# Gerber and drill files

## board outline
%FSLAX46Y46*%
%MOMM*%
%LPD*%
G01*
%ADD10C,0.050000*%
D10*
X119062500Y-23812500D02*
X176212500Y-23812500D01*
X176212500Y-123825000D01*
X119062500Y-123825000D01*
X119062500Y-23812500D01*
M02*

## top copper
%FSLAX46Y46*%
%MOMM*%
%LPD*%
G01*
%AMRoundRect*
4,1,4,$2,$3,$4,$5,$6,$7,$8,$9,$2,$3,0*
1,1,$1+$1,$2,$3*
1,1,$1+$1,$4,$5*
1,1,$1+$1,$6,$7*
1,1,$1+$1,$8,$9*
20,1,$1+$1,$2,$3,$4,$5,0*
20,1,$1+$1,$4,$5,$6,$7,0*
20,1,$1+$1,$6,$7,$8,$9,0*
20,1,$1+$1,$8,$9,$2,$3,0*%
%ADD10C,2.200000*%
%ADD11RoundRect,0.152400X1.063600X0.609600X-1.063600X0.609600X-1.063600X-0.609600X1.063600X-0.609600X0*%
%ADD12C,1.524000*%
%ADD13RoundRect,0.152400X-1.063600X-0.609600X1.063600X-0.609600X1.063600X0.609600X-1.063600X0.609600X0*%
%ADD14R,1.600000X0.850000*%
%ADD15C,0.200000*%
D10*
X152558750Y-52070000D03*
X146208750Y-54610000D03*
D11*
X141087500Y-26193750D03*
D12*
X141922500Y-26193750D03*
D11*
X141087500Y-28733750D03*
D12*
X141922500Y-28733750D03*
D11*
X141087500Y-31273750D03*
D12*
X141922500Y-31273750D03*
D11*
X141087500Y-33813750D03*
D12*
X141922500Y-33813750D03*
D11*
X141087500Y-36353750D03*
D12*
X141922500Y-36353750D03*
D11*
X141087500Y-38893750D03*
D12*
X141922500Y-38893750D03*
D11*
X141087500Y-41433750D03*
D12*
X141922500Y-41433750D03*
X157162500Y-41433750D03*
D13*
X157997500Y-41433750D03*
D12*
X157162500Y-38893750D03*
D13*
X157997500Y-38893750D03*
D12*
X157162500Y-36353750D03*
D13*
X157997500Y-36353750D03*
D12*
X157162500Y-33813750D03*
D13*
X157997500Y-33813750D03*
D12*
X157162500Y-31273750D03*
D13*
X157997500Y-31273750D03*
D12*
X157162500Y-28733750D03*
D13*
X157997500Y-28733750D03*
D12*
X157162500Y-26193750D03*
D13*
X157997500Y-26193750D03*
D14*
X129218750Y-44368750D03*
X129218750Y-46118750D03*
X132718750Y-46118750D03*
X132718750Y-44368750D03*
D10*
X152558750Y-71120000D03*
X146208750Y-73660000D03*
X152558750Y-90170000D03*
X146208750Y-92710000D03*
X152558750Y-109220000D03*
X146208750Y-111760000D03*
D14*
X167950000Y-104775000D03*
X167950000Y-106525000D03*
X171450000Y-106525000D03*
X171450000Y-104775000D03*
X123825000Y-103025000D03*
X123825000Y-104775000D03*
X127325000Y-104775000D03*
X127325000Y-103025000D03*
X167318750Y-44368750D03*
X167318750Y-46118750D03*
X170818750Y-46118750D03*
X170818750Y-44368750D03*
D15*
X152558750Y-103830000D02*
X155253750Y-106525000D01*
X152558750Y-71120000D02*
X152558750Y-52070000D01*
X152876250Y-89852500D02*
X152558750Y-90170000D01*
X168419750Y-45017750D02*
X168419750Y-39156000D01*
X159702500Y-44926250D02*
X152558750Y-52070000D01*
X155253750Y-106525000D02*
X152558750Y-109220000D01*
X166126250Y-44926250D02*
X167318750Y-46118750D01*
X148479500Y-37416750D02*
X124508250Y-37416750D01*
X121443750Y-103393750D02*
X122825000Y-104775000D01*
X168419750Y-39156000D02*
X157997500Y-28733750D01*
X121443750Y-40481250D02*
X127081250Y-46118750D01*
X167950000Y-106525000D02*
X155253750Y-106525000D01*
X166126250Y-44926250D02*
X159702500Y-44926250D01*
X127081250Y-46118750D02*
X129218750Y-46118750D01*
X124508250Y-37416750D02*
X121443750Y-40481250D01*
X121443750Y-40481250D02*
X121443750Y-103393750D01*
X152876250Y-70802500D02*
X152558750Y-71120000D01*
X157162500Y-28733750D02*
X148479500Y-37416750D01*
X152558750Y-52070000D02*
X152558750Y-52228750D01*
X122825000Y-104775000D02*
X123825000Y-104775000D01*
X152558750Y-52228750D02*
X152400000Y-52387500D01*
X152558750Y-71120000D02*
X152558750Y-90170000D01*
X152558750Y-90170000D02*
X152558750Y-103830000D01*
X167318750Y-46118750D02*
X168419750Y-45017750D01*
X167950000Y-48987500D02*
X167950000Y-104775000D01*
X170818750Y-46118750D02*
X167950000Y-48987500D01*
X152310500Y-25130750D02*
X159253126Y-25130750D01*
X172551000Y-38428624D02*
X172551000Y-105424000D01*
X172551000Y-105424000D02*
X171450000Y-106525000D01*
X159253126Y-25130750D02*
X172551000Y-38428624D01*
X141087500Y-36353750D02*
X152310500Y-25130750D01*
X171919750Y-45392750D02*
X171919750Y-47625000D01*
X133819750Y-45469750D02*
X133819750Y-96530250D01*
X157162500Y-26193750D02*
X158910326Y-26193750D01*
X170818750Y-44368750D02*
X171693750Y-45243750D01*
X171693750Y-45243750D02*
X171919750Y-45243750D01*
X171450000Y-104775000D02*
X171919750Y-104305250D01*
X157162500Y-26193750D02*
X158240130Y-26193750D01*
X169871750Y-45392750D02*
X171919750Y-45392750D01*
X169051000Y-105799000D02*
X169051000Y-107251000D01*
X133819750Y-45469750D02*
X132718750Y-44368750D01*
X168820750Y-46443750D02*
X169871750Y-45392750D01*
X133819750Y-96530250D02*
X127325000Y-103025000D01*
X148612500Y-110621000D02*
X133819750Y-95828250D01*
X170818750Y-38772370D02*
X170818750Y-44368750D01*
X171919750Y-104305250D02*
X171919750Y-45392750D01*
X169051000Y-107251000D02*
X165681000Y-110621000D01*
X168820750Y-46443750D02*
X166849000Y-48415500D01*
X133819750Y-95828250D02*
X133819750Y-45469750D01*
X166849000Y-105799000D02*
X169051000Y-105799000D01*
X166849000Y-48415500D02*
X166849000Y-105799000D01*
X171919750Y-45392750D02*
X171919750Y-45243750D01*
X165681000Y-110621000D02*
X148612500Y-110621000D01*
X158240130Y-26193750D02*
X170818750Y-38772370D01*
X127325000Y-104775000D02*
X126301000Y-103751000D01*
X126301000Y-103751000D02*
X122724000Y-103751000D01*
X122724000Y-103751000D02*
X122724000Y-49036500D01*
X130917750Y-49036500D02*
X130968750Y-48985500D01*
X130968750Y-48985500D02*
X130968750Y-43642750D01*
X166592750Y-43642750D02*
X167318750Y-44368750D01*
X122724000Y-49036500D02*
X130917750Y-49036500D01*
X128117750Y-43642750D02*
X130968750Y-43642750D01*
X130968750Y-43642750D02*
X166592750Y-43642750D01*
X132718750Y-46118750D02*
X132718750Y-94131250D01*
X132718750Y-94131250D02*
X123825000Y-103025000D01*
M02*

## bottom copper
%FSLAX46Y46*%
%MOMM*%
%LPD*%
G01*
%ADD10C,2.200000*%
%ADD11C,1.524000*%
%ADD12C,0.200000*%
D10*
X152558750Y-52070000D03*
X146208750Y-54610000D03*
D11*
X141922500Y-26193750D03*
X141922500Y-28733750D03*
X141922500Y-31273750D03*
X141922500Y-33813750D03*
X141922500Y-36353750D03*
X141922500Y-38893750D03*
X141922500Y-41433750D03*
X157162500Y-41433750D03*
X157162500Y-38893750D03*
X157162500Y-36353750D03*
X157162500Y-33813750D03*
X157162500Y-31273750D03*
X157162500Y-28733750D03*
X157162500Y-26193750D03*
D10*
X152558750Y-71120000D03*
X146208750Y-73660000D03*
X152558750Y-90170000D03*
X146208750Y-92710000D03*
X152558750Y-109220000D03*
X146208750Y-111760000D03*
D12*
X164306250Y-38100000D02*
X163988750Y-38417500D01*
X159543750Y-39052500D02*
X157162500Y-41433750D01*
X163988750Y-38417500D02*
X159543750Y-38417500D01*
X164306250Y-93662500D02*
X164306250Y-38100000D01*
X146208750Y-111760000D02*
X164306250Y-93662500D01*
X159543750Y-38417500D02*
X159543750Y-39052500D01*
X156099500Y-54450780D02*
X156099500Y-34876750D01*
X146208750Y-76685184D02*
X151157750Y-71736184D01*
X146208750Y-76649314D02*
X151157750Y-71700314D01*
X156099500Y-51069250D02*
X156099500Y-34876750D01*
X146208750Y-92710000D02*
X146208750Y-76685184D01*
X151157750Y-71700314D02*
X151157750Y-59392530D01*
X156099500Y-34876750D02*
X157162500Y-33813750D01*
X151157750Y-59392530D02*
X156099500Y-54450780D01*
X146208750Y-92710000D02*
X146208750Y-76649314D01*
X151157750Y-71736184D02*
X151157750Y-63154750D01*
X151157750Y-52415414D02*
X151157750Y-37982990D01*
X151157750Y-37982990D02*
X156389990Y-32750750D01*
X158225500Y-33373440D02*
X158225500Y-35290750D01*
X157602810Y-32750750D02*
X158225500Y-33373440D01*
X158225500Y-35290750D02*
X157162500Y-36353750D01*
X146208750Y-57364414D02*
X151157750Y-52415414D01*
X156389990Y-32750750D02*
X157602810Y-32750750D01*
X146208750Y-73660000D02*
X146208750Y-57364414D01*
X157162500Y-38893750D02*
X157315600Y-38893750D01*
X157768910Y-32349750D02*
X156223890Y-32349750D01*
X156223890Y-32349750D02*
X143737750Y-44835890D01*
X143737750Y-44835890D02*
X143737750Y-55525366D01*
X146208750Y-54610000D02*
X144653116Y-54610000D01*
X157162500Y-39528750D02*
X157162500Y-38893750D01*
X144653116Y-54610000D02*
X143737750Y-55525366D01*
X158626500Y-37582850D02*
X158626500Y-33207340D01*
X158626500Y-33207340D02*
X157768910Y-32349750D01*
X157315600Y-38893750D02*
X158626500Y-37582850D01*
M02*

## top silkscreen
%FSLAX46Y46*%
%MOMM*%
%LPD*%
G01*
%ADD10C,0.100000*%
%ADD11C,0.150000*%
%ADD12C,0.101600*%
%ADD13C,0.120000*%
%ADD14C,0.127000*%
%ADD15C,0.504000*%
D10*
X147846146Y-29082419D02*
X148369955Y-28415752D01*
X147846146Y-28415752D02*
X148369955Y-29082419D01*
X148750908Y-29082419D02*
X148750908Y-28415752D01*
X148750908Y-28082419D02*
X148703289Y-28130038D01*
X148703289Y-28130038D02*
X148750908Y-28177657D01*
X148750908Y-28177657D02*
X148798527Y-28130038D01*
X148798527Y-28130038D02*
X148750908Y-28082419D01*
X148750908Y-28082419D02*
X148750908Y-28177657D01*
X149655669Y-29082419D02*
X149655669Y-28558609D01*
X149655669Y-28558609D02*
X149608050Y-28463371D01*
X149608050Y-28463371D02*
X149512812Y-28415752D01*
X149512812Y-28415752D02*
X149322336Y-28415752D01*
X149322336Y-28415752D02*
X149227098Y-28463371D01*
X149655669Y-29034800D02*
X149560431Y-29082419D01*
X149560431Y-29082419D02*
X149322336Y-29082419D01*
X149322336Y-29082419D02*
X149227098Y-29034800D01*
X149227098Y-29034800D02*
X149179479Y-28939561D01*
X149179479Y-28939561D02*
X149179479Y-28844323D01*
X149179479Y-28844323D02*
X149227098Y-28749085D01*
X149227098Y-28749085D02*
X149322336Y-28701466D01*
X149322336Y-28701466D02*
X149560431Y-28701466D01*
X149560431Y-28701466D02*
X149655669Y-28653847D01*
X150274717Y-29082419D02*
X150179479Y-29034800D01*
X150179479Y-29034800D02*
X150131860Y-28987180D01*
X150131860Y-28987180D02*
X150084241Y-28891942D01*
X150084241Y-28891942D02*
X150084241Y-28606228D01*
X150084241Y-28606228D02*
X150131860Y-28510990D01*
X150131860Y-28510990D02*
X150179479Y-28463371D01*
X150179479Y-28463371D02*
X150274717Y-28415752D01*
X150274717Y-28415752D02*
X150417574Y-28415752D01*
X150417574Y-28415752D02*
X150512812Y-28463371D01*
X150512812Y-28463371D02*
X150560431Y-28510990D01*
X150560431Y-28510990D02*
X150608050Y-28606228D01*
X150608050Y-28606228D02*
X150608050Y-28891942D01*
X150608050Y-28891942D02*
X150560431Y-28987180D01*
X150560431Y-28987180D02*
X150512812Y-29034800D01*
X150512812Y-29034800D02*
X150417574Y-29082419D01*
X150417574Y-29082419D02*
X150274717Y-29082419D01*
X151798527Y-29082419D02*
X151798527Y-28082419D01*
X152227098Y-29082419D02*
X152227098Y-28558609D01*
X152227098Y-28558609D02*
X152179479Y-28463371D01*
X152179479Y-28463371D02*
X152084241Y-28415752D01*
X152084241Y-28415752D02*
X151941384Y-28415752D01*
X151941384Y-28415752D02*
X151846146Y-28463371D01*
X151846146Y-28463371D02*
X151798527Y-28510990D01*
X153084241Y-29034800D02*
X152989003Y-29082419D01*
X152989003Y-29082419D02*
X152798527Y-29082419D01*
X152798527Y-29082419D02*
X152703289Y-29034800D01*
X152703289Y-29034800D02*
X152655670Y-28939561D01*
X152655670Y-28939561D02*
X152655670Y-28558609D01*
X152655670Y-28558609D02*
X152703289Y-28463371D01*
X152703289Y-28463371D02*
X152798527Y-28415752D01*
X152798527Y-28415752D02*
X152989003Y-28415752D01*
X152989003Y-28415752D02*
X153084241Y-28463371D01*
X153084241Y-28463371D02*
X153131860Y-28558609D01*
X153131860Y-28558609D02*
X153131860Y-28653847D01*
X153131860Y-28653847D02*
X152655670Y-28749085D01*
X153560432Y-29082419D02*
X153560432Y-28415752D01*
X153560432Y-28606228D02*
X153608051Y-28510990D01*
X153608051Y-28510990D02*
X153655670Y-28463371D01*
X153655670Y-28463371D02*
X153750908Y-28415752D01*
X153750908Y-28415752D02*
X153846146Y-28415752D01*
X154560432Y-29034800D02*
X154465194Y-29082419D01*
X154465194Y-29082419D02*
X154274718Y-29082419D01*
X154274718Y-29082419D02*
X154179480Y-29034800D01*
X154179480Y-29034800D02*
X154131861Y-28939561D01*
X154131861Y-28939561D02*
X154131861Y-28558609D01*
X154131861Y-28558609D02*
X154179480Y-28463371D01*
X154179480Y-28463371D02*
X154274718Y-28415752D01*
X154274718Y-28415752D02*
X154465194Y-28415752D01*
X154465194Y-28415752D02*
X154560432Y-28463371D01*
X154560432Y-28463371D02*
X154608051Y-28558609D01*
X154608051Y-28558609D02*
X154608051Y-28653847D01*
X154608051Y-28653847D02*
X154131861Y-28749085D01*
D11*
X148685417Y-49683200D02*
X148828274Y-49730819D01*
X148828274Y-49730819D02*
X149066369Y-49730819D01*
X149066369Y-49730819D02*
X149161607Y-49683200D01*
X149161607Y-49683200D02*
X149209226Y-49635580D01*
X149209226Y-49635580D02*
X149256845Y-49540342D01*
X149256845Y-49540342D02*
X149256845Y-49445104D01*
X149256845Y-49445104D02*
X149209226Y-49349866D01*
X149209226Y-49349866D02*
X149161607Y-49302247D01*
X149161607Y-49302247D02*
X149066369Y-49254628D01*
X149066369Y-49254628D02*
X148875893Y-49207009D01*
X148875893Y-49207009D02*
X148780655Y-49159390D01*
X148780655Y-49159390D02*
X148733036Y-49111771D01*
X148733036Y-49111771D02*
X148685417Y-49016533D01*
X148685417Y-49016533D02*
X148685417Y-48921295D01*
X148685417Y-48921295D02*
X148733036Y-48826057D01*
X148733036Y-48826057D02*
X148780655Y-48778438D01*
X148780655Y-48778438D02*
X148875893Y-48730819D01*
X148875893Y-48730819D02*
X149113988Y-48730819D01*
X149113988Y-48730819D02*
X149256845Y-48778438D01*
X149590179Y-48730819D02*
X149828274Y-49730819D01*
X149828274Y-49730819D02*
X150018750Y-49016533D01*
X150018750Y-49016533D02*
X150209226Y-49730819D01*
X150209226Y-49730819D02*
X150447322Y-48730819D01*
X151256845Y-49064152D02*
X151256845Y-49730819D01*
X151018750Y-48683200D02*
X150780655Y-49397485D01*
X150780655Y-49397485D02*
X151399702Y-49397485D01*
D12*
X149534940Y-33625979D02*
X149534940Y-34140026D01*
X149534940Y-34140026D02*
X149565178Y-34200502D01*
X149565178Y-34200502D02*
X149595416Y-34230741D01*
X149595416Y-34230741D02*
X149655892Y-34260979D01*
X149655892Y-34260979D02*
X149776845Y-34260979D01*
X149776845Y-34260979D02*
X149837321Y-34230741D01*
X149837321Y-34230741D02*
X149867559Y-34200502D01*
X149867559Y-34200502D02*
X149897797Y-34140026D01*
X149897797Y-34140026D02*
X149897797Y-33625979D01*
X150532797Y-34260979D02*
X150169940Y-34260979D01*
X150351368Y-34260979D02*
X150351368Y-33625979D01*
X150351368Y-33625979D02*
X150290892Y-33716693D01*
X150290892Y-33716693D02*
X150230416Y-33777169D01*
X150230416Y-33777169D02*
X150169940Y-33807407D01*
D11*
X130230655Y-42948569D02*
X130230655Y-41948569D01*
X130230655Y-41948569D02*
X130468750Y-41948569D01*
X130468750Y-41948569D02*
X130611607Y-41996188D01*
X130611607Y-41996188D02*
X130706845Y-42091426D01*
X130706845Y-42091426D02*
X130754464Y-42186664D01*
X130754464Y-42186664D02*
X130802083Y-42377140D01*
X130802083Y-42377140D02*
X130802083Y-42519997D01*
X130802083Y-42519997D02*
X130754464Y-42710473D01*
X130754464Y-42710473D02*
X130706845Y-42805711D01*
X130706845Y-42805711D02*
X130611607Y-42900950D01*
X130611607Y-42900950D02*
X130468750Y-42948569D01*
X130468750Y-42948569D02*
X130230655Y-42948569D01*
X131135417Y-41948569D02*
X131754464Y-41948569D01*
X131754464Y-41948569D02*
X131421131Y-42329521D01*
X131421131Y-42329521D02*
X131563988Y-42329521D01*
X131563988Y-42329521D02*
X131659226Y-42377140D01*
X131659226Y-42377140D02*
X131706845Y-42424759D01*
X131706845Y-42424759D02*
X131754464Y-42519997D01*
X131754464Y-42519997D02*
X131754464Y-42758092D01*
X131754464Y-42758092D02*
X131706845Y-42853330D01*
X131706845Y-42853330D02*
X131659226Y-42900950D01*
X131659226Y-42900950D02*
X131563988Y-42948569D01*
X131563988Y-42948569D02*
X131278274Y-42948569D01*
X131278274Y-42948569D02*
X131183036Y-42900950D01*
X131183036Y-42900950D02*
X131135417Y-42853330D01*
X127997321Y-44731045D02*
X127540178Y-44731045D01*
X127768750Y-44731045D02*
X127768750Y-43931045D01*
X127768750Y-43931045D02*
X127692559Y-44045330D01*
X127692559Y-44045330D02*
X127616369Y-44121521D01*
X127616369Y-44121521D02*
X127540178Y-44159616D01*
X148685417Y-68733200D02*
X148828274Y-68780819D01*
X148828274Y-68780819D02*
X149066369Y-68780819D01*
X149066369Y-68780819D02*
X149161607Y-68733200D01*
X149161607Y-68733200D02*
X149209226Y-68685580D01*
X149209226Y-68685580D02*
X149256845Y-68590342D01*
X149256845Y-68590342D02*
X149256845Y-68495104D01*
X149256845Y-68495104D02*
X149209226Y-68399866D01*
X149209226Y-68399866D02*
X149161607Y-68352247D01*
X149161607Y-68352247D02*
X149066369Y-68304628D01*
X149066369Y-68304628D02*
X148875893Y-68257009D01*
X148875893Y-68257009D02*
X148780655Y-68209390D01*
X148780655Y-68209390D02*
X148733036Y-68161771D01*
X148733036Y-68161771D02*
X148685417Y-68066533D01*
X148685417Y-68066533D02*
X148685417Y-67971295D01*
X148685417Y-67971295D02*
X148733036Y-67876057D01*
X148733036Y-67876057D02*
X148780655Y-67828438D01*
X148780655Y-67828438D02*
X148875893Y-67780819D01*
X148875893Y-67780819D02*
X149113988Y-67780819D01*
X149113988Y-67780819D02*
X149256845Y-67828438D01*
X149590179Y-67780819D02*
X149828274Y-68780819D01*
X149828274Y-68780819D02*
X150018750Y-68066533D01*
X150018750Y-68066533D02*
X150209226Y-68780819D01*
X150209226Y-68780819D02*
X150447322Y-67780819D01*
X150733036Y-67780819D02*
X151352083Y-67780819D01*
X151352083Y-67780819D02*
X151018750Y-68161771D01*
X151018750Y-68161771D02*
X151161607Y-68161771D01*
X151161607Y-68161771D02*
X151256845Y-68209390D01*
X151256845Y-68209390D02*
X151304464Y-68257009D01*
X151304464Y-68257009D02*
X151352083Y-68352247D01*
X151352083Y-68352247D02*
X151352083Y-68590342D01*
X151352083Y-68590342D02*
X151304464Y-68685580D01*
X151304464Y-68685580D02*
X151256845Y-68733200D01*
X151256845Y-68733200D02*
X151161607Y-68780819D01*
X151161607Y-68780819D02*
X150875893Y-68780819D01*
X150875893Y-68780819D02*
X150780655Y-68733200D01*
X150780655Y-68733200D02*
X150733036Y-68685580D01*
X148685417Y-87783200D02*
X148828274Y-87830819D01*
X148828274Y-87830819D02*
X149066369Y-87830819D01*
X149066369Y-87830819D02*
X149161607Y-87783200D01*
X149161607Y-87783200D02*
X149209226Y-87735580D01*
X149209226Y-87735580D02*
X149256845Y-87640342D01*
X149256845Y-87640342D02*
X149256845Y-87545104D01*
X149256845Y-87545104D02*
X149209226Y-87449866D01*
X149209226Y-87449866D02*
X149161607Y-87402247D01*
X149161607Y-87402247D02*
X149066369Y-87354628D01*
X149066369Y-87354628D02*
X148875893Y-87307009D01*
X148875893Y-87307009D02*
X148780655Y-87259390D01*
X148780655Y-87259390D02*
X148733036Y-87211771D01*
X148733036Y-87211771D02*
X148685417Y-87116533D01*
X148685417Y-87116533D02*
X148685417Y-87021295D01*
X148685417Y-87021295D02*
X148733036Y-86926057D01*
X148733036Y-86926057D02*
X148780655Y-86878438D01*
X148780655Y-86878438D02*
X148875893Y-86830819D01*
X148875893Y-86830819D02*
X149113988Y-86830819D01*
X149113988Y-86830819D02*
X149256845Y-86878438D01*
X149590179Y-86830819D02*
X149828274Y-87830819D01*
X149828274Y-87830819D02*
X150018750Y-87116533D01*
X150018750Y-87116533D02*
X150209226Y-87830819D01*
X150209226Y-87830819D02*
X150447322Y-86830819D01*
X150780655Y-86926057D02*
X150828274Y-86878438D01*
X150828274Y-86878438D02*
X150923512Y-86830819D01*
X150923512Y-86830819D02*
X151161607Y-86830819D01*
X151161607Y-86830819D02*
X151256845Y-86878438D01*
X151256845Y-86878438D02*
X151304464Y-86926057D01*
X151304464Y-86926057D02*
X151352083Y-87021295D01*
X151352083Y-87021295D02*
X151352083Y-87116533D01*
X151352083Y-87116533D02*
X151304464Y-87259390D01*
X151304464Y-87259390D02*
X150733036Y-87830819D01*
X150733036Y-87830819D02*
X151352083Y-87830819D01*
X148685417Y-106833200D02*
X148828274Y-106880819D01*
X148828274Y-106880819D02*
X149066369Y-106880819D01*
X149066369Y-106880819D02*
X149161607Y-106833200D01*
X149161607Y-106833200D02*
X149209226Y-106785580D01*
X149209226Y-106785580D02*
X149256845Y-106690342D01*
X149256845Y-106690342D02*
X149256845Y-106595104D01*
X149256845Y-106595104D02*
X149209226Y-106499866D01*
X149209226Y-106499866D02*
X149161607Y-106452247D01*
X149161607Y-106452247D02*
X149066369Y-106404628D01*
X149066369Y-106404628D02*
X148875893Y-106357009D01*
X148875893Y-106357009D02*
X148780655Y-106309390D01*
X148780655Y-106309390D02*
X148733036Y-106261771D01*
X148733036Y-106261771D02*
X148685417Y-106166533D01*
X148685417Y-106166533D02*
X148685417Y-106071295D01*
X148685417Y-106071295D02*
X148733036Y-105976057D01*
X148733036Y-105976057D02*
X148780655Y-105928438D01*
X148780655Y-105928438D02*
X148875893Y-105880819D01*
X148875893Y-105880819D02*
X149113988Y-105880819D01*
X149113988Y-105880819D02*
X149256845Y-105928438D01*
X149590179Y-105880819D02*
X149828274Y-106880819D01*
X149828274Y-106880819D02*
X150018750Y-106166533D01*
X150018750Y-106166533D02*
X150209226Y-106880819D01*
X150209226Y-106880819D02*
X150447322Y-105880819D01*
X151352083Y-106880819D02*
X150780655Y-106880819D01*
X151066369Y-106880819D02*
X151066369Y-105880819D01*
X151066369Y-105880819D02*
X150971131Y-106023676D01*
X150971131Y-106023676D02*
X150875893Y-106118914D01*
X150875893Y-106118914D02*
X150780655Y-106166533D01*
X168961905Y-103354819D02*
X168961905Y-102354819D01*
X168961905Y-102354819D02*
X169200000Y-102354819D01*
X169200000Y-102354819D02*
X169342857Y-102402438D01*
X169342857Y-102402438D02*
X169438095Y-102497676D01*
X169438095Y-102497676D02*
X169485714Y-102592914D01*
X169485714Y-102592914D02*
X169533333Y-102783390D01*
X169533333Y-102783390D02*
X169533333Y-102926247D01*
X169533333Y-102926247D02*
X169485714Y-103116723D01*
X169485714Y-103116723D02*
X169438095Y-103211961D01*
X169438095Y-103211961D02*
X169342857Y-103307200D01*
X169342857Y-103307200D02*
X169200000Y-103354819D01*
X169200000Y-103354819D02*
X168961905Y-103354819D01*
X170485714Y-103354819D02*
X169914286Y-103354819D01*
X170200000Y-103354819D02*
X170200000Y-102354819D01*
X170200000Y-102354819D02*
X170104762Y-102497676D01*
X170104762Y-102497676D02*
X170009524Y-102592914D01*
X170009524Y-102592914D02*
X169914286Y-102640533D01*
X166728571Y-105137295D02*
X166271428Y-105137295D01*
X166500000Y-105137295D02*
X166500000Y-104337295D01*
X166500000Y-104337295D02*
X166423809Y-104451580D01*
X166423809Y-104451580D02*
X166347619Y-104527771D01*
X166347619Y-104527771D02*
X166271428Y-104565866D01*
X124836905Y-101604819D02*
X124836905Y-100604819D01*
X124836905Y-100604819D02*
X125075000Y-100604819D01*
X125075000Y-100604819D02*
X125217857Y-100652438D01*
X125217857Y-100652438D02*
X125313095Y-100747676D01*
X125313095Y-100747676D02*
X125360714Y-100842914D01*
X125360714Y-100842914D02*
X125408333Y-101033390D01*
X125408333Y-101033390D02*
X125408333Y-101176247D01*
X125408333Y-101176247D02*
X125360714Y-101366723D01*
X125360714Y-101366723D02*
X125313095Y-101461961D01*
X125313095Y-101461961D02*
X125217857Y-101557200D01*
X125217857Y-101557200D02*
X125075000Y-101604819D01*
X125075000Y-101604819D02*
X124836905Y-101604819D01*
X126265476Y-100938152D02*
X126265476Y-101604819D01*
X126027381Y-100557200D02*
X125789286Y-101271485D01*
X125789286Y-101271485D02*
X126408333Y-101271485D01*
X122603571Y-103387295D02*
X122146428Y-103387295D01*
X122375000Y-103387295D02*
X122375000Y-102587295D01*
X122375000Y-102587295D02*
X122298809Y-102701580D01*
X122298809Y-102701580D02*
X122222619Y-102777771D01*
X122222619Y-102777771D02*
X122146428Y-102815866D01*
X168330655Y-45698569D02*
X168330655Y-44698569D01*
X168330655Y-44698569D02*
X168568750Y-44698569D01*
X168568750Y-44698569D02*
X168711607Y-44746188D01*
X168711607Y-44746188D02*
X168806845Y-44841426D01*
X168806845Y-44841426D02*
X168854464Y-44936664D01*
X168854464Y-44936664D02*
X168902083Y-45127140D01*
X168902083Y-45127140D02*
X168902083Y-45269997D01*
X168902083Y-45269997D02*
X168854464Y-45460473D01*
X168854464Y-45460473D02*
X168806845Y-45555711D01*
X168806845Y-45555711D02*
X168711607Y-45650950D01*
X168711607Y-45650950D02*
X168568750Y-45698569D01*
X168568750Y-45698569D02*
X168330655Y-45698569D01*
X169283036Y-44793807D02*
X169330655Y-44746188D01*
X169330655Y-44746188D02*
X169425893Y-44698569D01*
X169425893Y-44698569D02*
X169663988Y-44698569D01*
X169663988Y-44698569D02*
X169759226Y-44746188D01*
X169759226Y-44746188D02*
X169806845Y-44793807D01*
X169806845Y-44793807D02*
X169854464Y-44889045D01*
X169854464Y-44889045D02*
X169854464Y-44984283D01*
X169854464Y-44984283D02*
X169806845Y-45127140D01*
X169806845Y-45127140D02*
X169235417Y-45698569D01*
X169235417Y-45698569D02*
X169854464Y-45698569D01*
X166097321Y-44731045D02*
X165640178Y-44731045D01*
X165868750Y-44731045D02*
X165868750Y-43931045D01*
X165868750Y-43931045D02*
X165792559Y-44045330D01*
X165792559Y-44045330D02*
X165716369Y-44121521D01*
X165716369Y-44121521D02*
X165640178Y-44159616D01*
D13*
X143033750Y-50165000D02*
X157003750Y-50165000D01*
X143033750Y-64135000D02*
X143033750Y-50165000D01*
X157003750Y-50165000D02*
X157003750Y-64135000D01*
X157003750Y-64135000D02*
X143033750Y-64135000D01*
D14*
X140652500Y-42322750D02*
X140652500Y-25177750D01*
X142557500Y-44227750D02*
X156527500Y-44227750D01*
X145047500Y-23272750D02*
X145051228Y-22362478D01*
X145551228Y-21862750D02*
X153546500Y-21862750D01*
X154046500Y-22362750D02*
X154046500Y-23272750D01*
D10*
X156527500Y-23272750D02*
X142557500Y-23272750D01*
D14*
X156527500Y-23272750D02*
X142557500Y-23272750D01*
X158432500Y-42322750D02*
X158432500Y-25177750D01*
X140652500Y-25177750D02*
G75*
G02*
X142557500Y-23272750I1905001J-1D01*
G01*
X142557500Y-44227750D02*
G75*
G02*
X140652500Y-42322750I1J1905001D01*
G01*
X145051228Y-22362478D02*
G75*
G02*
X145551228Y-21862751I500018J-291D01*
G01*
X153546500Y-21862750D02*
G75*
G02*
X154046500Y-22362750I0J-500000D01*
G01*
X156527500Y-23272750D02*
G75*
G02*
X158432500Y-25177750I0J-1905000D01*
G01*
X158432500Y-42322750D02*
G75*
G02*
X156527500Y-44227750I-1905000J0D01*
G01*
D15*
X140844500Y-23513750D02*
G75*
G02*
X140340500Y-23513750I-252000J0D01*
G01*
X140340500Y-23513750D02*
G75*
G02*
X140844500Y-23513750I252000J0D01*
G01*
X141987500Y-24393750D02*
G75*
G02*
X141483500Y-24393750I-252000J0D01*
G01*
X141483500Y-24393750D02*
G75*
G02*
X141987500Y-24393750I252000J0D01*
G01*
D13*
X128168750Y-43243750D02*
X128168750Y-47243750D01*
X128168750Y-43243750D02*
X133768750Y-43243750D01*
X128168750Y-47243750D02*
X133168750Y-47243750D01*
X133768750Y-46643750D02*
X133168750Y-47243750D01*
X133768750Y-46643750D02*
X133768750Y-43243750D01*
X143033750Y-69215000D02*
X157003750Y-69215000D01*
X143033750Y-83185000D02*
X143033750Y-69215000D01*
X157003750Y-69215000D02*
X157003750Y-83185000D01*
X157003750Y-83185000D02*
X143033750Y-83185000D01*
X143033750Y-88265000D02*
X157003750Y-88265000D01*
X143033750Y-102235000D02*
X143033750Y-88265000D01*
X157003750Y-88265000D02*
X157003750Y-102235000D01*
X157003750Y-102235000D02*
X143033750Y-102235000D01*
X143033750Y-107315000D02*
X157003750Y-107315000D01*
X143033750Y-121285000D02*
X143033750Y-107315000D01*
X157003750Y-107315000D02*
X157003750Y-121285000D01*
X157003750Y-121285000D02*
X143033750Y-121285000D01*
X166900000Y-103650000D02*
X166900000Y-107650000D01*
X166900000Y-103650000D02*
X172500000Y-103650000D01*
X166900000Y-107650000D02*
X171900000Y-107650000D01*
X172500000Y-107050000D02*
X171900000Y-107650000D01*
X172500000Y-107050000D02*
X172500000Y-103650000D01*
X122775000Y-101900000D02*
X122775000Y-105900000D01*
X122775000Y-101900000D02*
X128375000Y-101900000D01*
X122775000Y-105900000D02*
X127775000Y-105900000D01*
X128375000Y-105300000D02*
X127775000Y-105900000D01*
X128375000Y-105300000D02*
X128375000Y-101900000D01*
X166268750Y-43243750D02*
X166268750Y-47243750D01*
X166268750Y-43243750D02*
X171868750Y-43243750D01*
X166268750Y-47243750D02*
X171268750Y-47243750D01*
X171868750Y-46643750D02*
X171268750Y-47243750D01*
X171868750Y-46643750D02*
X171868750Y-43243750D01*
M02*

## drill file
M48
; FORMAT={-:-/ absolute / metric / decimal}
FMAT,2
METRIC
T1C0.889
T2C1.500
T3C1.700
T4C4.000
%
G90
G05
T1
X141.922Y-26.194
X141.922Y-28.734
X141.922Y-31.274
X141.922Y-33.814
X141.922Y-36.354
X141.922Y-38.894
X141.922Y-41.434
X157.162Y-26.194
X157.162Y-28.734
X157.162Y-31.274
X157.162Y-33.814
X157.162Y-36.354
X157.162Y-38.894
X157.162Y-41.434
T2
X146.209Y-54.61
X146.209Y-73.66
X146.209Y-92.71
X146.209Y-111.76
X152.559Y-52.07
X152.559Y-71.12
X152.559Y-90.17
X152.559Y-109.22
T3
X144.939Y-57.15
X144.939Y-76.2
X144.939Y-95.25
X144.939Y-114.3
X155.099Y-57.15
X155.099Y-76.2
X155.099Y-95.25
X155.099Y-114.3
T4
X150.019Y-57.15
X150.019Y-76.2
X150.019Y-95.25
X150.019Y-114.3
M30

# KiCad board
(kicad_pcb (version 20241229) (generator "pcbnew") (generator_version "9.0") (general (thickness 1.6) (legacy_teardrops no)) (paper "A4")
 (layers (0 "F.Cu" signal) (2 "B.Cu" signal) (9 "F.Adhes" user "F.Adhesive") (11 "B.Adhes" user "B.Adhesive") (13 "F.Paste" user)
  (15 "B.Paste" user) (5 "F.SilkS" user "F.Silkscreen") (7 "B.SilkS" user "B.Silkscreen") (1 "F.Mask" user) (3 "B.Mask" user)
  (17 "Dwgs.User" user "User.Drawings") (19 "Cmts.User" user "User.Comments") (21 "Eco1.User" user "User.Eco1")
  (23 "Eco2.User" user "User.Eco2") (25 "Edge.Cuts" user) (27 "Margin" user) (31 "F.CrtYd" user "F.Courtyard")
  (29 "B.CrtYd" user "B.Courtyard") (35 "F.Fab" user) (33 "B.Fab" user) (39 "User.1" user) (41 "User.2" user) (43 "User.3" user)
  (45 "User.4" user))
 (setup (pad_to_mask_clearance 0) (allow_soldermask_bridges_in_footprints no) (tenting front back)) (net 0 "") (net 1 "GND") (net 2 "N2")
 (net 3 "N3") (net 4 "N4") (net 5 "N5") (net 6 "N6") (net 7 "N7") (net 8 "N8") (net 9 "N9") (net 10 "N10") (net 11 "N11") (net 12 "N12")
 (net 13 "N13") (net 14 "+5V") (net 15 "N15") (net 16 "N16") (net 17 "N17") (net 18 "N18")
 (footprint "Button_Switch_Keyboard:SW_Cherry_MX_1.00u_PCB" (layer "F.Cu") (at 152.55875 52.07)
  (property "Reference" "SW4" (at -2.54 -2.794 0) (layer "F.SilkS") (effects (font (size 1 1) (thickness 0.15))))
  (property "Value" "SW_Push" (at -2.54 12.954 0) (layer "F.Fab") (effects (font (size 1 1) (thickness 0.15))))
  (fp_line (start -9.525 -1.905) (end 4.445 -1.905) (stroke (width 0.12) (type solid)) (layer "F.SilkS"))
  (fp_line (start -9.525 12.065) (end -9.525 -1.905) (stroke (width 0.12) (type solid)) (layer "F.SilkS"))
  (fp_line (start 4.445 -1.905) (end 4.445 12.065) (stroke (width 0.12) (type solid)) (layer "F.SilkS"))
  (fp_line (start 4.445 12.065) (end -9.525 12.065) (stroke (width 0.12) (type solid)) (layer "F.SilkS"))
  (pad "" np_thru_hole circle (at -7.62 5.08) (size 1.7 1.7) (drill 1.7) (layers "*.Cu" "*.Mask"))
  (pad "" np_thru_hole circle (at -2.54 5.08) (size 4 4) (drill 4) (layers "*.Cu" "*.Mask"))
  (pad "" np_thru_hole circle (at 2.54 5.08) (size 1.7 1.7) (drill 1.7) (layers "*.Cu" "*.Mask"))
  (pad "1" thru_hole circle (at 0 0) (size 2.2 2.2) (drill 1.5) (layers "*.Cu" "*.Mask") (remove_unused_layers no) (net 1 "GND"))
  (pad "2" thru_hole circle (at -6.35 2.54) (size 2.2 2.2) (drill 1.5) (layers "*.Cu" "*.Mask") (remove_unused_layers no) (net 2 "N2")))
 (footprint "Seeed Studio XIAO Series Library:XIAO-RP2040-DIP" (layer "F.Cu") (at 149.5425 33.81375)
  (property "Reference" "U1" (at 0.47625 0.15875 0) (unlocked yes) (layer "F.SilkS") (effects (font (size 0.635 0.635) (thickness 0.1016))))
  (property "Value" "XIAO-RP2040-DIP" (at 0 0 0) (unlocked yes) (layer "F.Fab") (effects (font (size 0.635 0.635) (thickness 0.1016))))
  (fp_line (start -8.89 8.509) (end -8.89 -8.636) (stroke (width 0.127) (type solid)) (layer "F.SilkS"))
  (fp_line (start -6.985 10.414) (end 6.985 10.414) (stroke (width 0.127) (type solid)) (layer "F.SilkS"))
  (fp_line (start -4.495 -10.541) (end -4.491272 -11.451272) (stroke (width 0.127) (type solid)) (layer "F.SilkS"))
  (fp_line (start -3.991272 -11.951) (end 4.004 -11.951) (stroke (width 0.127) (type solid)) (layer "F.SilkS"))
  (fp_line (start 4.504 -11.451) (end 4.504 -10.541) (stroke (width 0.127) (type solid)) (layer "F.SilkS"))
  (fp_line (start 6.985 -10.541) (end -6.985 -10.541) (stroke (width 0.1) (type solid)) (layer "F.SilkS"))
  (fp_line (start 6.985 -10.541) (end -6.985 -10.541) (stroke (width 0.127) (type solid)) (layer "F.SilkS"))
  (fp_line (start 8.89 8.509) (end 8.89 -8.636) (stroke (width 0.127) (type solid)) (layer "F.SilkS"))
  (fp_arc (start -8.89 -8.636) (mid -8.332038 -9.983038) (end -6.985 -10.541) (stroke (width 0.127) (type solid)) (layer "F.SilkS"))
  (fp_arc (start -6.985 10.414) (mid -8.332038 9.856038) (end -8.89 8.509) (stroke (width 0.127) (type solid)) (layer "F.SilkS"))
  (fp_arc (start -4.491272 -11.451272) (mid -4.344728 -11.80464) (end -3.991272 -11.951) (stroke (width 0.127) (type default))
   (layer "F.SilkS"))
  (fp_arc (start 4.004 -11.951) (mid 4.357553 -11.804553) (end 4.504 -11.451) (stroke (width 0.127) (type default)) (layer "F.SilkS"))
  (fp_arc (start 6.985 -10.541) (mid 8.332038 -9.983038) (end 8.89 -8.636) (stroke (width 0.127) (type solid)) (layer "F.SilkS"))
  (fp_arc (start 8.89 8.509) (mid 8.332038 9.856038) (end 6.985 10.414) (stroke (width 0.127) (type solid)) (layer "F.SilkS"))
  (fp_circle (center -8.95 -10.3) (end -8.95 -10.554) (stroke (width 0.5) (type solid)) (fill yes) (layer "F.SilkS"))
  (fp_circle (center -7.807 -9.42) (end -7.807 -9.674) (stroke (width 0.5) (type solid)) (fill yes) (layer "F.SilkS"))
  (pad "1" smd roundrect (at -8.455 -7.62 180) (size 2.432 1.524) (layers "F.Cu" "F.Mask") (roundrect_rratio 0.1) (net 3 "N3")
   (thermal_bridge_angle 45))
  (pad "1" thru_hole circle (at -7.62 -7.62 180) (size 1.524 1.524) (drill 0.889) (layers "*.Cu" "*.Mask") (remove_unused_layers no)
   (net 3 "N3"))
  (pad "2" smd roundrect (at -8.455 -5.08 180) (size 2.432 1.524) (layers "F.Cu" "F.Mask") (roundrect_rratio 0.1) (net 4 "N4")
   (thermal_bridge_angle 45))
  (pad "2" thru_hole circle (at -7.62 -5.08 180) (size 1.524 1.524) (drill 0.889) (layers "*.Cu" "*.Mask") (remove_unused_layers no)
   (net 4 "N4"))
  (pad "3" smd roundrect (at -8.455 -2.54 180) (size 2.432 1.524) (layers "F.Cu" "F.Mask") (roundrect_rratio 0.1) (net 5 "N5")
   (thermal_bridge_angle 45))
  (pad "3" thru_hole circle (at -7.62 -2.54 180) (size 1.524 1.524) (drill 0.889) (layers "*.Cu" "*.Mask") (remove_unused_layers no)
   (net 5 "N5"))
  (pad "4" smd roundrect (at -8.455 0 180) (size 2.432 1.524) (layers "F.Cu" "F.Mask") (roundrect_rratio 0.1) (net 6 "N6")
   (thermal_bridge_angle 45))
  (pad "4" thru_hole circle (at -7.62 0 180) (size 1.524 1.524) (drill 0.889) (layers "*.Cu" "*.Mask") (remove_unused_layers no)
   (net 6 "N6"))
  (pad "5" smd roundrect (at -8.455 2.54 180) (size 2.432 1.524) (layers "F.Cu" "F.Mask") (roundrect_rratio 0.1) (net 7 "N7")
   (thermal_bridge_angle 45))
  (pad "5" thru_hole circle (at -7.62 2.54 180) (size 1.524 1.524) (drill 0.889) (layers "*.Cu" "*.Mask") (remove_unused_layers no)
   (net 7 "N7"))
  (pad "6" smd roundrect (at -8.455 5.08 180) (size 2.432 1.524) (layers "F.Cu" "F.Mask") (roundrect_rratio 0.1) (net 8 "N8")
   (thermal_bridge_angle 45))
  (pad "6" thru_hole circle (at -7.62 5.08 180) (size 1.524 1.524) (drill 0.889) (layers "*.Cu" "*.Mask") (remove_unused_layers no)
   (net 8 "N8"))
  (pad "7" smd roundrect (at -8.455 7.62 180) (size 2.432 1.524) (layers "F.Cu" "F.Mask") (roundrect_rratio 0.1) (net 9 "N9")
   (thermal_bridge_angle 45))
  (pad "7" thru_hole circle (at -7.62 7.62 180) (size 1.524 1.524) (drill 0.889) (layers "*.Cu" "*.Mask") (remove_unused_layers no)
   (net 9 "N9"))
  (pad "8" thru_hole circle (at 7.62 7.62) (size 1.524 1.524) (drill 0.889) (layers "*.Cu" "*.Mask") (remove_unused_layers no)
   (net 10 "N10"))
  (pad "8" smd roundrect (at 8.455 7.62) (size 2.432 1.524) (layers "F.Cu" "F.Mask") (roundrect_rratio 0.1) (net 10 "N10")
   (thermal_bridge_angle 45))
  (pad "9" thru_hole circle (at 7.62 5.08) (size 1.524 1.524) (drill 0.889) (layers "*.Cu" "*.Mask") (remove_unused_layers no) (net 2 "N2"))
  (pad "9" smd roundrect (at 8.455 5.08) (size 2.432 1.524) (layers "F.Cu" "F.Mask") (roundrect_rratio 0.1) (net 2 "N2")
   (thermal_bridge_angle 45))
  (pad "10" thru_hole circle (at 7.62 2.54) (size 1.524 1.524) (drill 0.889) (layers "*.Cu" "*.Mask") (remove_unused_layers no)
   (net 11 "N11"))
  (pad "10" smd roundrect (at 8.455 2.54) (size 2.432 1.524) (layers "F.Cu" "F.Mask") (roundrect_rratio 0.1) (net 11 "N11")
   (thermal_bridge_angle 45))
  (pad "11" thru_hole circle (at 7.62 0) (size 1.524 1.524) (drill 0.889) (layers "*.Cu" "*.Mask") (remove_unused_layers no) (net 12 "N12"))
  (pad "11" smd roundrect (at 8.455 0) (size 2.432 1.524) (layers "F.Cu" "F.Mask") (roundrect_rratio 0.1) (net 12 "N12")
   (thermal_bridge_angle 45))
  (pad "12" thru_hole circle (at 7.62 -2.54) (size 1.524 1.524) (drill 0.889) (layers "*.Cu" "*.Mask") (remove_unused_layers no)
   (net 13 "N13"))
  (pad "12" smd roundrect (at 8.455 -2.54) (size 2.432 1.524) (layers "F.Cu" "F.Mask") (roundrect_rratio 0.1) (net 13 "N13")
   (thermal_bridge_angle 45))
  (pad "13" thru_hole circle (at 7.62 -5.08) (size 1.524 1.524) (drill 0.889) (layers "*.Cu" "*.Mask") (remove_unused_layers no)
   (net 1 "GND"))
  (pad "13" smd roundrect (at 8.455 -5.08) (size 2.432 1.524) (layers "F.Cu" "F.Mask") (roundrect_rratio 0.1) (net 1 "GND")
   (thermal_bridge_angle 45))
  (pad "14" thru_hole circle (at 7.62 -7.62) (size 1.524 1.524) (drill 0.889) (layers "*.Cu" "*.Mask") (remove_unused_layers no)
   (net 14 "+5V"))
  (pad "14" smd roundrect (at 8.455 -7.62) (size 2.432 1.524) (layers "F.Cu" "F.Mask") (roundrect_rratio 0.1) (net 14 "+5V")
   (thermal_bridge_angle 45)))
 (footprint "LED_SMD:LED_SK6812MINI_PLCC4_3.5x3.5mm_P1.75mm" (layer "F.Cu") (at 130.96875 45.24375)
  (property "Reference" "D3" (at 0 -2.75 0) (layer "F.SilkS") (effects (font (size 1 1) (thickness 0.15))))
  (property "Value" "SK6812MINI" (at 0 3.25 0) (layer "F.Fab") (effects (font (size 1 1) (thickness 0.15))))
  (fp_line (start -2.8 -2) (end -2.8 2) (stroke (width 0.12) (type default)) (layer "F.SilkS"))
  (fp_line (start -2.8 -2) (end 2.8 -2) (stroke (width 0.12) (type solid)) (layer "F.SilkS"))
  (fp_line (start -2.8 2) (end 2.2 2) (stroke (width 0.12) (type solid)) (layer "F.SilkS"))
  (fp_line (start 2.8 1.4) (end 2.2 2) (stroke (width 0.12) (type default)) (layer "F.SilkS"))
  (fp_line (start 2.8 1.4) (end 2.8 -2) (stroke (width 0.12) (type solid)) (layer "F.SilkS"))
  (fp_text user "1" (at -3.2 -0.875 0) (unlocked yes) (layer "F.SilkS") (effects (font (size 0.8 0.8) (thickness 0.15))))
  (pad "1" smd rect (at -1.75 -0.875) (size 1.6 0.85) (layers "F.Cu" "F.Mask" "F.Paste") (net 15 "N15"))
  (pad "2" smd rect (at -1.75 0.875) (size 1.6 0.85) (layers "F.Cu" "F.Mask" "F.Paste") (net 1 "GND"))
  (pad "3" smd rect (at 1.75 0.875) (size 1.6 0.85) (layers "F.Cu" "F.Mask" "F.Paste") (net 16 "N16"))
  (pad "4" smd rect (at 1.75 -0.875) (size 1.6 0.85) (layers "F.Cu" "F.Mask" "F.Paste") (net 14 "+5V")))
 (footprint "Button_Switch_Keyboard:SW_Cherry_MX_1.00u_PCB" (layer "F.Cu") (at 152.55875 71.12)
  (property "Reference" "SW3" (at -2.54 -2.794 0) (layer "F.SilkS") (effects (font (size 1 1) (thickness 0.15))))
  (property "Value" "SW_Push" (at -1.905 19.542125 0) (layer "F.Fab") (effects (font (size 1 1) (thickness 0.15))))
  (fp_line (start -9.525 -1.905) (end 4.445 -1.905) (stroke (width 0.12) (type solid)) (layer "F.SilkS"))
  (fp_line (start -9.525 12.065) (end -9.525 -1.905) (stroke (width 0.12) (type solid)) (layer "F.SilkS"))
  (fp_line (start 4.445 -1.905) (end 4.445 12.065) (stroke (width 0.12) (type solid)) (layer "F.SilkS"))
  (fp_line (start 4.445 12.065) (end -9.525 12.065) (stroke (width 0.12) (type solid)) (layer "F.SilkS"))
  (pad "" np_thru_hole circle (at -7.62 5.08) (size 1.7 1.7) (drill 1.7) (layers "*.Cu" "*.Mask"))
  (pad "" np_thru_hole circle (at -2.54 5.08) (size 4 4) (drill 4) (layers "*.Cu" "*.Mask"))
  (pad "" np_thru_hole circle (at 2.54 5.08) (size 1.7 1.7) (drill 1.7) (layers "*.Cu" "*.Mask"))
  (pad "1" thru_hole circle (at 0 0) (size 2.2 2.2) (drill 1.5) (layers "*.Cu" "*.Mask") (remove_unused_layers no) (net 1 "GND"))
  (pad "2" thru_hole circle (at -6.35 2.54) (size 2.2 2.2) (drill 1.5) (layers "*.Cu" "*.Mask") (remove_unused_layers no) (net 11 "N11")))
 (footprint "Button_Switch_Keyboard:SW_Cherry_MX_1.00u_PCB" (layer "F.Cu") (at 152.55875 90.17)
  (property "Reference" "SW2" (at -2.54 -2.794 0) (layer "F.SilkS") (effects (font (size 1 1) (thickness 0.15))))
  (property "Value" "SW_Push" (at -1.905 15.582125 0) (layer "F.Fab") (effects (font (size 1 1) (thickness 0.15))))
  (fp_line (start -9.525 -1.905) (end 4.445 -1.905) (stroke (width 0.12) (type solid)) (layer "F.SilkS"))
  (fp_line (start -9.525 12.065) (end -9.525 -1.905) (stroke (width 0.12) (type solid)) (layer "F.SilkS"))
  (fp_line (start 4.445 -1.905) (end 4.445 12.065) (stroke (width 0.12) (type solid)) (layer "F.SilkS"))
  (fp_line (start 4.445 12.065) (end -9.525 12.065) (stroke (width 0.12) (type solid)) (layer "F.SilkS"))
  (pad "" np_thru_hole circle (at -7.62 5.08) (size 1.7 1.7) (drill 1.7) (layers "*.Cu" "*.Mask"))
  (pad "" np_thru_hole circle (at -2.54 5.08) (size 4 4) (drill 4) (layers "*.Cu" "*.Mask"))
  (pad "" np_thru_hole circle (at 2.54 5.08) (size 1.7 1.7) (drill 1.7) (layers "*.Cu" "*.Mask"))
  (pad "1" thru_hole circle (at 0 0) (size 2.2 2.2) (drill 1.5) (layers "*.Cu" "*.Mask") (remove_unused_layers no) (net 1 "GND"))
  (pad "2" thru_hole circle (at -6.35 2.54) (size 2.2 2.2) (drill 1.5) (layers "*.Cu" "*.Mask") (remove_unused_layers no) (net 12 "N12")))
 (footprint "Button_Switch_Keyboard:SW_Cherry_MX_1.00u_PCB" (layer "F.Cu") (at 152.55875 109.22)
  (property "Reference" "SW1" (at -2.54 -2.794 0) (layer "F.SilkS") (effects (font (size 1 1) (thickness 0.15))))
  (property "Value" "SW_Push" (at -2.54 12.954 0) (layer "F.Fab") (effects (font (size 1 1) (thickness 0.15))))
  (fp_line (start -9.525 -1.905) (end 4.445 -1.905) (stroke (width 0.12) (type solid)) (layer "F.SilkS"))
  (fp_line (start -9.525 12.065) (end -9.525 -1.905) (stroke (width 0.12) (type solid)) (layer "F.SilkS"))
  (fp_line (start 4.445 -1.905) (end 4.445 12.065) (stroke (width 0.12) (type solid)) (layer "F.SilkS"))
  (fp_line (start 4.445 12.065) (end -9.525 12.065) (stroke (width 0.12) (type solid)) (layer "F.SilkS"))
  (pad "" np_thru_hole circle (at -7.62 5.08) (size 1.7 1.7) (drill 1.7) (layers "*.Cu" "*.Mask"))
  (pad "" np_thru_hole circle (at -2.54 5.08) (size 4 4) (drill 4) (layers "*.Cu" "*.Mask"))
  (pad "" np_thru_hole circle (at 2.54 5.08) (size 1.7 1.7) (drill 1.7) (layers "*.Cu" "*.Mask"))
  (pad "1" thru_hole circle (at 0 0) (size 2.2 2.2) (drill 1.5) (layers "*.Cu" "*.Mask") (remove_unused_layers no) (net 1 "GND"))
  (pad "2" thru_hole circle (at -6.35 2.54) (size 2.2 2.2) (drill 1.5) (layers "*.Cu" "*.Mask") (remove_unused_layers no) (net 10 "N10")))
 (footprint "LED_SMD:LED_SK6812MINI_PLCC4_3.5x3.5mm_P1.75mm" (layer "F.Cu") (at 169.7 105.65)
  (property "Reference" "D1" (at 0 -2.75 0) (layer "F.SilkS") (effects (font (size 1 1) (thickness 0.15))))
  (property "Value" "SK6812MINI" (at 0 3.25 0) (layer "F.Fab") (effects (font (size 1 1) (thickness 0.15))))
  (fp_line (start -2.8 -2) (end -2.8 2) (stroke (width 0.12) (type default)) (layer "F.SilkS"))
  (fp_line (start -2.8 -2) (end 2.8 -2) (stroke (width 0.12) (type solid)) (layer "F.SilkS"))
  (fp_line (start -2.8 2) (end 2.2 2) (stroke (width 0.12) (type solid)) (layer "F.SilkS"))
  (fp_line (start 2.8 1.4) (end 2.2 2) (stroke (width 0.12) (type default)) (layer "F.SilkS"))
  (fp_line (start 2.8 1.4) (end 2.8 -2) (stroke (width 0.12) (type solid)) (layer "F.SilkS"))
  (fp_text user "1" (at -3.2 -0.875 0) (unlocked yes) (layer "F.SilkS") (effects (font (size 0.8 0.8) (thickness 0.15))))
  (pad "1" smd rect (at -1.75 -0.875) (size 1.6 0.85) (layers "F.Cu" "F.Mask" "F.Paste") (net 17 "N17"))
  (pad "2" smd rect (at -1.75 0.875) (size 1.6 0.85) (layers "F.Cu" "F.Mask" "F.Paste") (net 1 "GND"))
  (pad "3" smd rect (at 1.75 0.875) (size 1.6 0.85) (layers "F.Cu" "F.Mask" "F.Paste") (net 7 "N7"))
  (pad "4" smd rect (at 1.75 -0.875) (size 1.6 0.85) (layers "F.Cu" "F.Mask" "F.Paste") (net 14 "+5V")))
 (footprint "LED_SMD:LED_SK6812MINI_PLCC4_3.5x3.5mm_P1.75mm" (layer "F.Cu") (at 125.575 103.9)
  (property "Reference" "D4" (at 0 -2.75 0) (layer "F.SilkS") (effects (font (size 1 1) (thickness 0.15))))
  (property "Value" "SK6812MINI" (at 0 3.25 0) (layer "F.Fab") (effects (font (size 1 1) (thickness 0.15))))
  (fp_line (start -2.8 -2) (end -2.8 2) (stroke (width 0.12) (type default)) (layer "F.SilkS"))
  (fp_line (start -2.8 -2) (end 2.8 -2) (stroke (width 0.12) (type solid)) (layer "F.SilkS"))
  (fp_line (start -2.8 2) (end 2.2 2) (stroke (width 0.12) (type solid)) (layer "F.SilkS"))
  (fp_line (start 2.8 1.4) (end 2.2 2) (stroke (width 0.12) (type default)) (layer "F.SilkS"))
  (fp_line (start 2.8 1.4) (end 2.8 -2) (stroke (width 0.12) (type solid)) (layer "F.SilkS"))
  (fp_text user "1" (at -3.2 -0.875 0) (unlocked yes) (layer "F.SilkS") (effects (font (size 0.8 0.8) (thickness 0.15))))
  (pad "1" smd rect (at -1.75 -0.875) (size 1.6 0.85) (layers "F.Cu" "F.Mask" "F.Paste") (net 16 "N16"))
  (pad "2" smd rect (at -1.75 0.875) (size 1.6 0.85) (layers "F.Cu" "F.Mask" "F.Paste") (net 1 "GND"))
  (pad "3" smd rect (at 1.75 0.875) (size 1.6 0.85) (layers "F.Cu" "F.Mask" "F.Paste") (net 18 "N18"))
  (pad "4" smd rect (at 1.75 -0.875) (size 1.6 0.85) (layers "F.Cu" "F.Mask" "F.Paste") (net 14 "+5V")))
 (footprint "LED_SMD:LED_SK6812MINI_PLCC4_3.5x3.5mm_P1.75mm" (layer "F.Cu") (at 169.06875 45.24375)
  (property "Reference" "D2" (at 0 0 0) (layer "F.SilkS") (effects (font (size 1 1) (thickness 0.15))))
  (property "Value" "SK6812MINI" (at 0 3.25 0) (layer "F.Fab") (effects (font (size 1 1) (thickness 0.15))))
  (fp_line (start -2.8 -2) (end -2.8 2) (stroke (width 0.12) (type default)) (layer "F.SilkS"))
  (fp_line (start -2.8 -2) (end 2.8 -2) (stroke (width 0.12) (type solid)) (layer "F.SilkS"))
  (fp_line (start -2.8 2) (end 2.2 2) (stroke (width 0.12) (type solid)) (layer "F.SilkS"))
  (fp_line (start 2.8 1.4) (end 2.2 2) (stroke (width 0.12) (type default)) (layer "F.SilkS"))
  (fp_line (start 2.8 1.4) (end 2.8 -2) (stroke (width 0.12) (type solid)) (layer "F.SilkS"))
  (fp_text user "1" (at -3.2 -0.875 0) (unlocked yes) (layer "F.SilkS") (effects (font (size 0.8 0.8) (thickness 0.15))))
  (pad "1" smd rect (at -1.75 -0.875) (size 1.6 0.85) (layers "F.Cu" "F.Mask" "F.Paste") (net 18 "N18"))
  (pad "2" smd rect (at -1.75 0.875) (size 1.6 0.85) (layers "F.Cu" "F.Mask" "F.Paste") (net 1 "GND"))
  (pad "3" smd rect (at 1.75 0.875) (size 1.6 0.85) (layers "F.Cu" "F.Mask" "F.Paste") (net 17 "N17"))
  (pad "4" smd rect (at 1.75 -0.875) (size 1.6 0.85) (layers "F.Cu" "F.Mask" "F.Paste") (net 14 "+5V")))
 (gr_rect (start 119.0625 23.8125) (end 176.2125 123.825) (stroke (width 0.05) (type default)) (fill no) (layer "Edge.Cuts"))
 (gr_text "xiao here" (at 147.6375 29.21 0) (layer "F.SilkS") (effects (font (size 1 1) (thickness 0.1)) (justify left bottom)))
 (segment (start 152.55875 103.83) (end 155.25375 106.525) (width 0.2) (layer "F.Cu") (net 1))
 (segment (start 152.55875 71.12) (end 152.55875 52.07) (width 0.2) (layer "F.Cu") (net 1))
 (segment (start 152.87625 89.8525) (end 152.55875 90.17) (width 0.2) (layer "F.Cu") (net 1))
 (segment (start 168.41975 45.01775) (end 168.41975 39.156) (width 0.2) (layer "F.Cu") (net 1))
 (segment (start 159.7025 44.92625) (end 152.55875 52.07) (width 0.2) (layer "F.Cu") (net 1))
 (segment (start 155.25375 106.525) (end 152.55875 109.22) (width 0.2) (layer "F.Cu") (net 1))
 (segment (start 166.12625 44.92625) (end 167.31875 46.11875) (width 0.2) (layer "F.Cu") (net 1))
 (segment (start 148.4795 37.41675) (end 124.50825 37.41675) (width 0.2) (layer "F.Cu") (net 1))
 (segment (start 121.44375 103.39375) (end 122.825 104.775) (width 0.2) (layer "F.Cu") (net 1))
 (segment (start 168.41975 39.156) (end 157.9975 28.73375) (width 0.2) (layer "F.Cu") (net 1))
 (segment (start 121.44375 40.48125) (end 127.08125 46.11875) (width 0.2) (layer "F.Cu") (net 1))
 (segment (start 167.95 106.525) (end 155.25375 106.525) (width 0.2) (layer "F.Cu") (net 1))
 (segment (start 166.12625 44.92625) (end 159.7025 44.92625) (width 0.2) (layer "F.Cu") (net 1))
 (segment (start 127.08125 46.11875) (end 129.21875 46.11875) (width 0.2) (layer "F.Cu") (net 1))
 (segment (start 124.50825 37.41675) (end 121.44375 40.48125) (width 0.2) (layer "F.Cu") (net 1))
 (segment (start 121.44375 40.48125) (end 121.44375 103.39375) (width 0.2) (layer "F.Cu") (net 1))
 (segment (start 152.87625 70.8025) (end 152.55875 71.12) (width 0.2) (layer "F.Cu") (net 1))
 (segment (start 157.1625 28.73375) (end 148.4795 37.41675) (width 0.2) (layer "F.Cu") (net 1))
 (segment (start 152.55875 52.07) (end 152.55875 52.22875) (width 0.2) (layer "F.Cu") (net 1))
 (segment (start 122.825 104.775) (end 123.825 104.775) (width 0.2) (layer "F.Cu") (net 1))
 (segment (start 152.55875 52.22875) (end 152.4 52.3875) (width 0.2) (layer "F.Cu") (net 1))
 (segment (start 152.55875 71.12) (end 152.55875 90.17) (width 0.2) (layer "F.Cu") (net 1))
 (segment (start 152.55875 90.17) (end 152.55875 103.83) (width 0.2) (layer "F.Cu") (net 1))
 (segment (start 167.31875 46.11875) (end 168.41975 45.01775) (width 0.2) (layer "F.Cu") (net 1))
 (segment (start 167.95 48.9875) (end 167.95 104.775) (width 0.2) (layer "F.Cu") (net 17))
 (segment (start 170.81875 46.11875) (end 167.95 48.9875) (width 0.2) (layer "F.Cu") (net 17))
 (segment (start 152.3105 25.13075) (end 159.253126 25.13075) (width 0.2) (layer "F.Cu") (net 7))
 (segment (start 172.551 38.428624) (end 172.551 105.424) (width 0.2) (layer "F.Cu") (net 7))
 (segment (start 172.551 105.424) (end 171.45 106.525) (width 0.2) (layer "F.Cu") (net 7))
 (segment (start 159.253126 25.13075) (end 172.551 38.428624) (width 0.2) (layer "F.Cu") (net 7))
 (segment (start 141.0875 36.35375) (end 152.3105 25.13075) (width 0.2) (layer "F.Cu") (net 7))
 (segment (start 171.91975 45.39275) (end 171.91975 47.625) (width 0.2) (layer "F.Cu") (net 14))
 (segment (start 133.81975 45.46975) (end 133.81975 96.53025) (width 0.2) (layer "F.Cu") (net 14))
 (segment (start 157.1625 26.19375) (end 158.910326 26.19375) (width 0.2) (layer "F.Cu") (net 14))
 (segment (start 170.81875 44.36875) (end 171.69375 45.24375) (width 0.2) (layer "F.Cu") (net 14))
 (segment (start 171.69375 45.24375) (end 171.91975 45.24375) (width 0.2) (layer "F.Cu") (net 14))
 (segment (start 171.45 104.775) (end 171.91975 104.30525) (width 0.2) (layer "F.Cu") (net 14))
 (segment (start 157.1625 26.19375) (end 158.24013 26.19375) (width 0.2) (layer "F.Cu") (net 14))
 (segment (start 169.87175 45.39275) (end 171.91975 45.39275) (width 0.2) (layer "F.Cu") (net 14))
 (segment (start 169.051 105.799) (end 169.051 107.251) (width 0.2) (layer "F.Cu") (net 14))
 (segment (start 133.81975 45.46975) (end 132.71875 44.36875) (width 0.2) (layer "F.Cu") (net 14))
 (segment (start 168.82075 46.44375) (end 169.87175 45.39275) (width 0.2) (layer "F.Cu") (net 14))
 (segment (start 133.81975 96.53025) (end 127.325 103.025) (width 0.2) (layer "F.Cu") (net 14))
 (segment (start 148.6125 110.621) (end 133.81975 95.82825) (width 0.2) (layer "F.Cu") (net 14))
 (segment (start 170.81875 38.77237) (end 170.81875 44.36875) (width 0.2) (layer "F.Cu") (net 14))
 (segment (start 171.91975 104.30525) (end 171.91975 45.39275) (width 0.2) (layer "F.Cu") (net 14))
 (segment (start 169.051 107.251) (end 165.681 110.621) (width 0.2) (layer "F.Cu") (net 14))
 (segment (start 168.82075 46.44375) (end 166.849 48.4155) (width 0.2) (layer "F.Cu") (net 14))
 (segment (start 133.81975 95.82825) (end 133.81975 45.46975) (width 0.2) (layer "F.Cu") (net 14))
 (segment (start 166.849 105.799) (end 169.051 105.799) (width 0.2) (layer "F.Cu") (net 14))
 (segment (start 166.849 48.4155) (end 166.849 105.799) (width 0.2) (layer "F.Cu") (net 14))
 (segment (start 171.91975 45.39275) (end 171.91975 45.24375) (width 0.2) (layer "F.Cu") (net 14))
 (segment (start 165.681 110.621) (end 148.6125 110.621) (width 0.2) (layer "F.Cu") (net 14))
 (segment (start 158.24013 26.19375) (end 170.81875 38.77237) (width 0.2) (layer "F.Cu") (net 14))
 (segment (start 127.325 104.775) (end 126.301 103.751) (width 0.2) (layer "F.Cu") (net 18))
 (segment (start 126.301 103.751) (end 122.724 103.751) (width 0.2) (layer "F.Cu") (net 18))
 (segment (start 122.724 103.751) (end 122.724 49.0365) (width 0.2) (layer "F.Cu") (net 18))
 (segment (start 130.91775 49.0365) (end 130.96875 48.9855) (width 0.2) (layer "F.Cu") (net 18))
 (segment (start 130.96875 48.9855) (end 130.96875 43.64275) (width 0.2) (layer "F.Cu") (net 18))
 (segment (start 166.59275 43.64275) (end 167.31875 44.36875) (width 0.2) (layer "F.Cu") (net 18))
 (segment (start 122.724 49.0365) (end 130.91775 49.0365) (width 0.2) (layer "F.Cu") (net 18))
 (segment (start 128.11775 43.64275) (end 130.96875 43.64275) (width 0.2) (layer "F.Cu") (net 18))
 (segment (start 130.96875 43.64275) (end 166.59275 43.64275) (width 0.2) (layer "F.Cu") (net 18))
 (segment (start 132.71875 46.11875) (end 132.71875 94.13125) (width 0.2) (layer "F.Cu") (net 16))
 (segment (start 132.71875 94.13125) (end 123.825 103.025) (width 0.2) (layer "F.Cu") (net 16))
 (segment (start 164.30625 38.1) (end 163.98875 38.4175) (width 0.2) (layer "B.Cu") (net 10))
 (segment (start 159.54375 39.0525) (end 157.1625 41.43375) (width 0.2) (layer "B.Cu") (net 10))
 (segment (start 163.98875 38.4175) (end 159.54375 38.4175) (width 0.2) (layer "B.Cu") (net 10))
 (segment (start 164.30625 93.6625) (end 164.30625 38.1) (width 0.2) (layer "B.Cu") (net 10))
 (segment (start 146.20875 111.76) (end 164.30625 93.6625) (width 0.2) (layer "B.Cu") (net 10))
 (segment (start 159.54375 38.4175) (end 159.54375 39.0525) (width 0.2) (layer "B.Cu") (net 10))
 (segment (start 156.0995 54.45078) (end 156.0995 34.87675) (width 0.2) (layer "B.Cu") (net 12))
 (segment (start 146.20875 76.685184) (end 151.15775 71.736184) (width 0.2) (layer "B.Cu") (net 12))
 (segment (start 146.20875 76.649314) (end 151.15775 71.700314) (width 0.2) (layer "B.Cu") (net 12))
 (segment (start 156.0995 51.06925) (end 156.0995 34.87675) (width 0.2) (layer "B.Cu") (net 12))
 (segment (start 146.20875 92.71) (end 146.20875 76.685184) (width 0.2) (layer "B.Cu") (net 12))
 (segment (start 151.15775 71.700314) (end 151.15775 59.39253) (width 0.2) (layer "B.Cu") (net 12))
 (segment (start 156.0995 34.87675) (end 157.1625 33.81375) (width 0.2) (layer "B.Cu") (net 12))
 (segment (start 151.15775 59.39253) (end 156.0995 54.45078) (width 0.2) (layer "B.Cu") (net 12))
 (segment (start 146.20875 92.71) (end 146.20875 76.649314) (width 0.2) (layer "B.Cu") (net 12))
 (segment (start 151.15775 71.736184) (end 151.15775 63.15475) (width 0.2) (layer "B.Cu") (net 12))
 (segment (start 151.15775 52.415414) (end 151.15775 37.98299) (width 0.2) (layer "B.Cu") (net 11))
 (segment (start 151.15775 37.98299) (end 156.38999 32.75075) (width 0.2) (layer "B.Cu") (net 11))
 (segment (start 158.2255 33.37344) (end 158.2255 35.29075) (width 0.2) (layer "B.Cu") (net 11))
 (segment (start 157.60281 32.75075) (end 158.2255 33.37344) (width 0.2) (layer "B.Cu") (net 11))
 (segment (start 158.2255 35.29075) (end 157.1625 36.35375) (width 0.2) (layer "B.Cu") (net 11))
 (segment (start 146.20875 57.364414) (end 151.15775 52.415414) (width 0.2) (layer "B.Cu") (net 11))
 (segment (start 156.38999 32.75075) (end 157.60281 32.75075) (width 0.2) (layer "B.Cu") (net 11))
 (segment (start 146.20875 73.66) (end 146.20875 57.364414) (width 0.2) (layer "B.Cu") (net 11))
 (segment (start 157.1625 38.89375) (end 157.3156 38.89375) (width 0.2) (layer "B.Cu") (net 2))
 (segment (start 157.76891 32.34975) (end 156.22389 32.34975) (width 0.2) (layer "B.Cu") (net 2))
 (segment (start 156.22389 32.34975) (end 143.73775 44.83589) (width 0.2) (layer "B.Cu") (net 2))
 (segment (start 143.73775 44.83589) (end 143.73775 55.525366) (width 0.2) (layer "B.Cu") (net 2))
 (segment (start 146.20875 54.61) (end 144.653116 54.61) (width 0.2) (layer "B.Cu") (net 2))
 (segment (start 157.1625 39.52875) (end 157.1625 38.89375) (width 0.2) (layer "B.Cu") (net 2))
 (segment (start 144.653116 54.61) (end 143.73775 55.525366) (width 0.2) (layer "B.Cu") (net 2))
 (segment (start 158.6265 37.58285) (end 158.6265 33.20734) (width 0.2) (layer "B.Cu") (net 2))
 (segment (start 158.6265 33.20734) (end 157.76891 32.34975) (width 0.2) (layer "B.Cu") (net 2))
 (segment (start 157.3156 38.89375) (end 158.6265 37.58285) (width 0.2) (layer "B.Cu") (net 2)))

